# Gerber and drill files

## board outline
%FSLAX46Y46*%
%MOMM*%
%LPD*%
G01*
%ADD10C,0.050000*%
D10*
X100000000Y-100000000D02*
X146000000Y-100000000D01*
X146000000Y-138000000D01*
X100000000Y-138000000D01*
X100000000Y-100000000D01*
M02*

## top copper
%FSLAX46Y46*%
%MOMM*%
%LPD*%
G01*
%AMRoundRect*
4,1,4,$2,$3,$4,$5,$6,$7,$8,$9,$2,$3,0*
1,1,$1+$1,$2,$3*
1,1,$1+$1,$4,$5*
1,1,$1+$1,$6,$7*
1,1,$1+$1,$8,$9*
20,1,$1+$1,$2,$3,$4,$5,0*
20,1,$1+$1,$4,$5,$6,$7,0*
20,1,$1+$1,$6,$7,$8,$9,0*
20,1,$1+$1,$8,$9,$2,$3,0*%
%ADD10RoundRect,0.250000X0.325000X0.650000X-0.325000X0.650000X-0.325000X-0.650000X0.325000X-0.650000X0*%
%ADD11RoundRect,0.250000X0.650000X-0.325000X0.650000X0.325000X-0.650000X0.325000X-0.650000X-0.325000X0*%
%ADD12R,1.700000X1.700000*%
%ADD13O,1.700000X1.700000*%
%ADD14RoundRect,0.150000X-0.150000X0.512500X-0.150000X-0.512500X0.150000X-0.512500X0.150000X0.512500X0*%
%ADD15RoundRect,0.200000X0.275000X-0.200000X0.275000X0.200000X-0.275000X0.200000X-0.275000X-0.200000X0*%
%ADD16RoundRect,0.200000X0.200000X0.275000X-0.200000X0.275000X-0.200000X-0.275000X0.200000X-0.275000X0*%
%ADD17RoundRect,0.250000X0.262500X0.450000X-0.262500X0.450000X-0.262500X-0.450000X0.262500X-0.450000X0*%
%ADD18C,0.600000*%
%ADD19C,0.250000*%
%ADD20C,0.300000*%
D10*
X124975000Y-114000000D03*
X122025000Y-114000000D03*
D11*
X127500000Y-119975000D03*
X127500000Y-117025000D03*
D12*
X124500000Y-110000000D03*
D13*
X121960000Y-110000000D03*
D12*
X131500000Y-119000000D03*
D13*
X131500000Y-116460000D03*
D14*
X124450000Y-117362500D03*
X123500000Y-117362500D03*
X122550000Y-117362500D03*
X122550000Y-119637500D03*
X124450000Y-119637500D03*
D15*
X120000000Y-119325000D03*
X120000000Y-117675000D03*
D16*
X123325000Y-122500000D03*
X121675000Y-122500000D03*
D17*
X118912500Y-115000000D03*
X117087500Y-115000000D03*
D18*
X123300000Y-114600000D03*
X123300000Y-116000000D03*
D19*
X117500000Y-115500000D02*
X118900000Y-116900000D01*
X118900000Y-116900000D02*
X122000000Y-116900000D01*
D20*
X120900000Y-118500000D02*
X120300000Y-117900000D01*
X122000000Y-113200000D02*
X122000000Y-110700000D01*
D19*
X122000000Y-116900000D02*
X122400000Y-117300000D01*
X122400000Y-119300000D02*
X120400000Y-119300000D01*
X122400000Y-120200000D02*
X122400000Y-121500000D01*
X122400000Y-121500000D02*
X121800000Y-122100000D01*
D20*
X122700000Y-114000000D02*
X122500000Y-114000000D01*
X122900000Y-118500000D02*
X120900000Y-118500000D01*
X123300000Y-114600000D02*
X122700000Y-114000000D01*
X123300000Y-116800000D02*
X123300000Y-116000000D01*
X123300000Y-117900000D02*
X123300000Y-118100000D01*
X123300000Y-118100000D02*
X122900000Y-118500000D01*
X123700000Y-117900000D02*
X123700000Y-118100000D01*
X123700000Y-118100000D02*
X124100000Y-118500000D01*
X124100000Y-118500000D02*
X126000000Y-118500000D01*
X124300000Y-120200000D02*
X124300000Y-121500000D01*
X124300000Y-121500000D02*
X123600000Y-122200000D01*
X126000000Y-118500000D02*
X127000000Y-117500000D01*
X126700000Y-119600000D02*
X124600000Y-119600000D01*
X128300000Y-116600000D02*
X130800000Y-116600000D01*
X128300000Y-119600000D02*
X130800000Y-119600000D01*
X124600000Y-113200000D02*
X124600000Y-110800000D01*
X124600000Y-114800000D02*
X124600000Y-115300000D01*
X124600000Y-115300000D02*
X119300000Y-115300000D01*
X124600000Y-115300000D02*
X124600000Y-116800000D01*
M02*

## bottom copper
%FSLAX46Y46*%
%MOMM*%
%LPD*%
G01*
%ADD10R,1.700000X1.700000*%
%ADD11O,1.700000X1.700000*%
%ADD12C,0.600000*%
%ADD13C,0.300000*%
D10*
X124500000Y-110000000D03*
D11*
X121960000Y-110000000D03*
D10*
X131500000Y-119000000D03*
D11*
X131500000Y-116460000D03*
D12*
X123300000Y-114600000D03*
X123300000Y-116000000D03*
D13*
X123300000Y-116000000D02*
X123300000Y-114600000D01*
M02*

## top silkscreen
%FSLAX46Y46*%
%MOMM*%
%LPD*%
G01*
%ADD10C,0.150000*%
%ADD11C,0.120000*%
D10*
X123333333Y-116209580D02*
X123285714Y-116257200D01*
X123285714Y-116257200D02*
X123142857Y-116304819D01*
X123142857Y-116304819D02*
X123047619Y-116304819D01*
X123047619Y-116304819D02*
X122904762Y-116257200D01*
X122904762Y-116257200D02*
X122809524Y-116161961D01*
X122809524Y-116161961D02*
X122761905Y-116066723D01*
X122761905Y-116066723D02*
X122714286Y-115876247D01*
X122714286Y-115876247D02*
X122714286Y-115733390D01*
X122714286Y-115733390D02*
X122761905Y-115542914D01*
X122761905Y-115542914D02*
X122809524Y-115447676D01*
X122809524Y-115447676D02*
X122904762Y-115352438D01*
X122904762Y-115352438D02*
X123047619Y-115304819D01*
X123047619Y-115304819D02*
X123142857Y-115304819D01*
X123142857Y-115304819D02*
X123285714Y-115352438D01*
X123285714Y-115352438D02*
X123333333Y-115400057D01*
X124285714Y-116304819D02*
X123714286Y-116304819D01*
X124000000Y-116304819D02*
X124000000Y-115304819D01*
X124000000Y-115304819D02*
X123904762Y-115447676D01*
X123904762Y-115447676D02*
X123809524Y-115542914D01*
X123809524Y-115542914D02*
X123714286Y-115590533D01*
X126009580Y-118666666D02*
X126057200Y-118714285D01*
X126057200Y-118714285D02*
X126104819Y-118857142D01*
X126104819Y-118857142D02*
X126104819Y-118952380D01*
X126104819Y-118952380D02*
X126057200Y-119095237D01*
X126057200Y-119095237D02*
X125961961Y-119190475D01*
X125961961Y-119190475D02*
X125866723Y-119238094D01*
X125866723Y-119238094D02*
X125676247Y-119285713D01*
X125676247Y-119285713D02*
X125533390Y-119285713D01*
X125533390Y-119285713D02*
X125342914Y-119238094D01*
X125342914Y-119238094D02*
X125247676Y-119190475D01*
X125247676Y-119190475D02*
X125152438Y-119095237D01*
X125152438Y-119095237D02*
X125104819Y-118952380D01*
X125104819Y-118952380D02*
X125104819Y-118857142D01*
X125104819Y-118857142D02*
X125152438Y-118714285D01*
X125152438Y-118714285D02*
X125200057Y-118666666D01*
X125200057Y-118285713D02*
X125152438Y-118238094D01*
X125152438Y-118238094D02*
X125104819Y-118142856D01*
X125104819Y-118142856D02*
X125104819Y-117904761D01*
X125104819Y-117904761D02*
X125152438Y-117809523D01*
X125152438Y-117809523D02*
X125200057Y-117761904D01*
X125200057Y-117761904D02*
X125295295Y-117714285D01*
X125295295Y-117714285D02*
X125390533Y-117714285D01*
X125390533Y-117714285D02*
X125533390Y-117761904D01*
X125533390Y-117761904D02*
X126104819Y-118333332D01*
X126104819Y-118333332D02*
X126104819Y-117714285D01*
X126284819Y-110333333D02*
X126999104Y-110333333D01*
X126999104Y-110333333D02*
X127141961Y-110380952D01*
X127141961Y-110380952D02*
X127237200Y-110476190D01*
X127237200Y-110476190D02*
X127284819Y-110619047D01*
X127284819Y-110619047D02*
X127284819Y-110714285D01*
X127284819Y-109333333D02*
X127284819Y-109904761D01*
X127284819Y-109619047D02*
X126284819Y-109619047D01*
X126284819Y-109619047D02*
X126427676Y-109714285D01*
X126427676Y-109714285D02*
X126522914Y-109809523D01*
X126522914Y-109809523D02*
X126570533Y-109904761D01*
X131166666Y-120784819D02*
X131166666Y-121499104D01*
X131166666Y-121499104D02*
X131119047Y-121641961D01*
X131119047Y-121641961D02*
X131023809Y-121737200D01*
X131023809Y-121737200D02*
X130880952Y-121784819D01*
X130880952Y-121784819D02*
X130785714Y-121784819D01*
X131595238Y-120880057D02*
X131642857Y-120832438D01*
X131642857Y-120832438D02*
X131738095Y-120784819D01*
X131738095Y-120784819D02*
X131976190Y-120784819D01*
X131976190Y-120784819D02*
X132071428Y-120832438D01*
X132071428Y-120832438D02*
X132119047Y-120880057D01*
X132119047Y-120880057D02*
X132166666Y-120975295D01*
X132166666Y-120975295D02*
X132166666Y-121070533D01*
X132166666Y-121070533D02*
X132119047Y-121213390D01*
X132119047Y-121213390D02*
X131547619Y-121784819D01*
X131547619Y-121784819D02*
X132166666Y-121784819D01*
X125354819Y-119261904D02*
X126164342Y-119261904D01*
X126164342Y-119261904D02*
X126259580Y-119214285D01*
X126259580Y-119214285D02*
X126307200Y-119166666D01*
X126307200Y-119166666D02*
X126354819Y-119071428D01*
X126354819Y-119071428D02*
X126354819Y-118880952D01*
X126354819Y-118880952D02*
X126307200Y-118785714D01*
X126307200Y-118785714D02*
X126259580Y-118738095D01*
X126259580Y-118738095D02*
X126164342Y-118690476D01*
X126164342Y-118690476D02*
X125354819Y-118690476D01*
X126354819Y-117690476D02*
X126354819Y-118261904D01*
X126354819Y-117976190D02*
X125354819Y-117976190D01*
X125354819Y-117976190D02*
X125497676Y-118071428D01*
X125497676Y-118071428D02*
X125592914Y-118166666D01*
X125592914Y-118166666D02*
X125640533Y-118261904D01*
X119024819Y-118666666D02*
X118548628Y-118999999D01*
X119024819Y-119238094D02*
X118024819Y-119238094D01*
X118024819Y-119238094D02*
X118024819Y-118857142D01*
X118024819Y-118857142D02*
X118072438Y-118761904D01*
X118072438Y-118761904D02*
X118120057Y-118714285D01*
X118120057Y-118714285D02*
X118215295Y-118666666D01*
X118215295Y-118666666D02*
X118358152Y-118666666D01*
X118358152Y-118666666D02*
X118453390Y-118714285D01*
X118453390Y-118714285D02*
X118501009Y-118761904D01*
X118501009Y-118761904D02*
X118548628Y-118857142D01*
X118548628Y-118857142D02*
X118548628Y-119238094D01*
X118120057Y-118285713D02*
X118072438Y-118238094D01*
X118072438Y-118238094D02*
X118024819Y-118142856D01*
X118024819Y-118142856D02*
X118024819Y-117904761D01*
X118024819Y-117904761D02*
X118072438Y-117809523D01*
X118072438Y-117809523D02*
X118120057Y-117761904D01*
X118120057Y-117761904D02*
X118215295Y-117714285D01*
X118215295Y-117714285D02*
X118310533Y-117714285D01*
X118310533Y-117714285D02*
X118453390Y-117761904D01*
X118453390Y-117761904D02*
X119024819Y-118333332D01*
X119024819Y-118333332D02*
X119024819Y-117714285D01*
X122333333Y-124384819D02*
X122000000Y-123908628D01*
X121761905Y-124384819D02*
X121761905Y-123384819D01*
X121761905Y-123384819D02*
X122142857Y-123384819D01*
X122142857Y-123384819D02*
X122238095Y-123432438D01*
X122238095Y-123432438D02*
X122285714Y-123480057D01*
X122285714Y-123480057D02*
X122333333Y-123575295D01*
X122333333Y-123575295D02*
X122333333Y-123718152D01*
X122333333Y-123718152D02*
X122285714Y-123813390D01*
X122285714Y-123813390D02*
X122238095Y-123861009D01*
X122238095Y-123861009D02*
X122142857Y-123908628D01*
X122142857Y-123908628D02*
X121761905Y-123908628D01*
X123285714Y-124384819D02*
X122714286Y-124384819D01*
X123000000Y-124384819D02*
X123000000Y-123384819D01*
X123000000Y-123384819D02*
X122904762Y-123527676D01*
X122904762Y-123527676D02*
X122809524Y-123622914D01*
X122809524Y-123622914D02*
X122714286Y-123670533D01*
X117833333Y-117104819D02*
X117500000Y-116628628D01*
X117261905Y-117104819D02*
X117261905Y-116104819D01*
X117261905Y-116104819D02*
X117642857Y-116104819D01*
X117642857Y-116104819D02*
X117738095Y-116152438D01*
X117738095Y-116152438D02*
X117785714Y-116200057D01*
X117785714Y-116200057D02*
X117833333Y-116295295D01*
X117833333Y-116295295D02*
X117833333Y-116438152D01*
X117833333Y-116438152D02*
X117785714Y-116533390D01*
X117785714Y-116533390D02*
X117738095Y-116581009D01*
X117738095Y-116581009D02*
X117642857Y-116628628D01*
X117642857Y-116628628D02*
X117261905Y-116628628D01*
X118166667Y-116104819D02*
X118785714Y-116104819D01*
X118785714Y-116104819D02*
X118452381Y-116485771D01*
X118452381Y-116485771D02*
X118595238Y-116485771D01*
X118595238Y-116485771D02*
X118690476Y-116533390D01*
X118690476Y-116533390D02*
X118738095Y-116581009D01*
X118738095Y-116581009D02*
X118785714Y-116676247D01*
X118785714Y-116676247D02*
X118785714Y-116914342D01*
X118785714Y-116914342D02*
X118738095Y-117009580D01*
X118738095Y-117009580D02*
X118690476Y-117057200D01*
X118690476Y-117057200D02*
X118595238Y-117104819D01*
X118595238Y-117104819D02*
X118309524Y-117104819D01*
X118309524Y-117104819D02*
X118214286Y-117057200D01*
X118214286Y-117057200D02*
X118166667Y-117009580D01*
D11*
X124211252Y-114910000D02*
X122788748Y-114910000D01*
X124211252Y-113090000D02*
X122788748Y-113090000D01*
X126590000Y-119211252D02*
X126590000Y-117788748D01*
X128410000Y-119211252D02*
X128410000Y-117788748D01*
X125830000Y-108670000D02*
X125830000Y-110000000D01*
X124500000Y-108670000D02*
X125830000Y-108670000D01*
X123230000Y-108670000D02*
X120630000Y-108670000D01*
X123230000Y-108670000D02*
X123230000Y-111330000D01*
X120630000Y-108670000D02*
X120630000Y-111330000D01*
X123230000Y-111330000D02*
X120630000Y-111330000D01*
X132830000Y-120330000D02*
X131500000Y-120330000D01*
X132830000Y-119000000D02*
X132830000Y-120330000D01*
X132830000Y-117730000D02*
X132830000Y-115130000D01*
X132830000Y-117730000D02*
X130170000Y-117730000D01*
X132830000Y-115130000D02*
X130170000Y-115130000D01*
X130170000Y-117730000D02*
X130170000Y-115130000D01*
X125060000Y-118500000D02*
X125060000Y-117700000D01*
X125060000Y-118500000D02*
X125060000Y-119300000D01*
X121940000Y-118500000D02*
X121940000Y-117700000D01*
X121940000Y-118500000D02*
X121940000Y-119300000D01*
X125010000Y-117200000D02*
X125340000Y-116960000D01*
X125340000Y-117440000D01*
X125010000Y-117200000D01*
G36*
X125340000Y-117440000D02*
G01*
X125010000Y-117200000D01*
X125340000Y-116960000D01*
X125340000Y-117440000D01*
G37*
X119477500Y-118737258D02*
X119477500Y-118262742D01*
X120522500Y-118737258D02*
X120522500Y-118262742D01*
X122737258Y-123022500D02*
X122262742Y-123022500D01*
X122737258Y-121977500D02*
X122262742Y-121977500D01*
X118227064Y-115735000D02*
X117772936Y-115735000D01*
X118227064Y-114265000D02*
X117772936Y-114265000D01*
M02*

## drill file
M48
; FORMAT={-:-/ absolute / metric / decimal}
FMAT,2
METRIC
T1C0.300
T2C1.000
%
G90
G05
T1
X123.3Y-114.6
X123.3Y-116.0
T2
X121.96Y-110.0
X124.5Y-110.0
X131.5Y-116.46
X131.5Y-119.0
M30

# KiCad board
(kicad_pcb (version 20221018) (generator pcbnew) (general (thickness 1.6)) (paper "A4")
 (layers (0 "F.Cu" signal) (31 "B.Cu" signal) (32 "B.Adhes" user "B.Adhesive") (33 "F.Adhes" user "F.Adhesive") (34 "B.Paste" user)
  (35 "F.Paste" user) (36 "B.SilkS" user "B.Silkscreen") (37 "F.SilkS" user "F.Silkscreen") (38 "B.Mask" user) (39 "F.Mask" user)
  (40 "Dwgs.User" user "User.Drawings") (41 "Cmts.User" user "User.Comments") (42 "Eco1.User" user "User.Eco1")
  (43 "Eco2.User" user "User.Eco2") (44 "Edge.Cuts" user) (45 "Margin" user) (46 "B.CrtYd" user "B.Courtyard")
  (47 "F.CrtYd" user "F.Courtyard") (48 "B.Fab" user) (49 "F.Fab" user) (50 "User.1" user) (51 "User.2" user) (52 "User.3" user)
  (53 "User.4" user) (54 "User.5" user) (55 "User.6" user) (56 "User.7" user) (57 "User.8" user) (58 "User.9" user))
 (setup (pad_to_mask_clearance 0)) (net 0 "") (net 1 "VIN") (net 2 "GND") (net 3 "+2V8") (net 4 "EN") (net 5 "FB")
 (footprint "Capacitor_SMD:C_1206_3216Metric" (layer "F.Cu") (at 123.5 114 180)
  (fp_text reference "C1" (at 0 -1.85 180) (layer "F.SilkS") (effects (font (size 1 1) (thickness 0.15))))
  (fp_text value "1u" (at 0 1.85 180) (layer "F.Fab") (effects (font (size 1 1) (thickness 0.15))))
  (fp_line (start -0.711252 -0.91) (end 0.711252 -0.91) (stroke (width 0.12) (type solid)) (layer "F.SilkS"))
  (fp_line (start -0.711252 0.91) (end 0.711252 0.91) (stroke (width 0.12) (type solid)) (layer "F.SilkS"))
  (pad "1" smd roundrect (at -1.475 0 180) (size 1.15 1.8) (layers "F.Cu" "F.Paste" "F.Mask") (roundrect_rratio 0.217391) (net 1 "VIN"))
  (pad "2" smd roundrect (at 1.475 0 180) (size 1.15 1.8) (layers "F.Cu" "F.Paste" "F.Mask") (roundrect_rratio 0.217391) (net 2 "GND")))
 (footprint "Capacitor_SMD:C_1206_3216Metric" (layer "F.Cu") (at 127.5 118.5 90)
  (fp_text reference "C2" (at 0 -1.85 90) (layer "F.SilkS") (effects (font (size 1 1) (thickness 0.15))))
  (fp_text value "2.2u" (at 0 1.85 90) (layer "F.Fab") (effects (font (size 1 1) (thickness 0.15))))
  (fp_line (start -0.711252 -0.91) (end 0.711252 -0.91) (stroke (width 0.12) (type solid)) (layer "F.SilkS"))
  (fp_line (start -0.711252 0.91) (end 0.711252 0.91) (stroke (width 0.12) (type solid)) (layer "F.SilkS"))
  (pad "1" smd roundrect (at -1.475 0 90) (size 1.15 1.8) (layers "F.Cu" "F.Paste" "F.Mask") (roundrect_rratio 0.217391) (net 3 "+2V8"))
  (pad "2" smd roundrect (at 1.475 0 90) (size 1.15 1.8) (layers "F.Cu" "F.Paste" "F.Mask") (roundrect_rratio 0.217391) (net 2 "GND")))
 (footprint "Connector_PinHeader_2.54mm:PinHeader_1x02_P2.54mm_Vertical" (layer "F.Cu") (at 124.5 110 -90)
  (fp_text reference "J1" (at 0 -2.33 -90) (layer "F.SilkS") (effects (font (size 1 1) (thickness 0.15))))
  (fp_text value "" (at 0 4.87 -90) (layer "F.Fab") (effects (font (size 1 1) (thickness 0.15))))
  (fp_line (start -1.33 -1.33) (end 0 -1.33) (stroke (width 0.12) (type solid)) (layer "F.SilkS"))
  (fp_line (start -1.33 0) (end -1.33 -1.33) (stroke (width 0.12) (type solid)) (layer "F.SilkS"))
  (fp_line (start -1.33 1.27) (end -1.33 3.87) (stroke (width 0.12) (type solid)) (layer "F.SilkS"))
  (fp_line (start -1.33 1.27) (end 1.33 1.27) (stroke (width 0.12) (type solid)) (layer "F.SilkS"))
  (fp_line (start -1.33 3.87) (end 1.33 3.87) (stroke (width 0.12) (type solid)) (layer "F.SilkS"))
  (fp_line (start 1.33 1.27) (end 1.33 3.87) (stroke (width 0.12) (type solid)) (layer "F.SilkS"))
  (pad "1" thru_hole rect (at 0 0 270) (size 1.7 1.7) (drill 1) (layers "*.Cu" "*.Mask") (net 1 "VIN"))
  (pad "2" thru_hole oval (at 0 2.54 270) (size 1.7 1.7) (drill 1) (layers "*.Cu" "*.Mask") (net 2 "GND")))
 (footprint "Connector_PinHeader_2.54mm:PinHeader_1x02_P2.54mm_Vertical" (layer "F.Cu") (at 131.5 119 180)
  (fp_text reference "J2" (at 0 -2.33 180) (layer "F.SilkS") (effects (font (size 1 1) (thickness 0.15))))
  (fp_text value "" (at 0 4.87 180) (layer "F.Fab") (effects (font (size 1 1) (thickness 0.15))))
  (fp_line (start -1.33 -1.33) (end 0 -1.33) (stroke (width 0.12) (type solid)) (layer "F.SilkS"))
  (fp_line (start -1.33 0) (end -1.33 -1.33) (stroke (width 0.12) (type solid)) (layer "F.SilkS"))
  (fp_line (start -1.33 1.27) (end -1.33 3.87) (stroke (width 0.12) (type solid)) (layer "F.SilkS"))
  (fp_line (start -1.33 1.27) (end 1.33 1.27) (stroke (width 0.12) (type solid)) (layer "F.SilkS"))
  (fp_line (start -1.33 3.87) (end 1.33 3.87) (stroke (width 0.12) (type solid)) (layer "F.SilkS"))
  (fp_line (start 1.33 1.27) (end 1.33 3.87) (stroke (width 0.12) (type solid)) (layer "F.SilkS"))
  (pad "1" thru_hole rect (at 0 0 180) (size 1.7 1.7) (drill 1) (layers "*.Cu" "*.Mask") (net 3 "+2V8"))
  (pad "2" thru_hole oval (at 0 2.54 180) (size 1.7 1.7) (drill 1) (layers "*.Cu" "*.Mask") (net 2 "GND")))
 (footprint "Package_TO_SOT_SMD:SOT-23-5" (layer "F.Cu") (at 123.5 118.5 -90)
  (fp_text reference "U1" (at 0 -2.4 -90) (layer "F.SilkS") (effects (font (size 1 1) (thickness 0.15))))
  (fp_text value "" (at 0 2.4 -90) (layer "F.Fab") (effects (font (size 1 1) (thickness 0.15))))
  (fp_line (start 0 -1.56) (end -0.8 -1.56) (stroke (width 0.12) (type solid)) (layer "F.SilkS"))
  (fp_line (start 0 -1.56) (end 0.8 -1.56) (stroke (width 0.12) (type solid)) (layer "F.SilkS"))
  (fp_line (start 0 1.56) (end -0.8 1.56) (stroke (width 0.12) (type solid)) (layer "F.SilkS"))
  (fp_line (start 0 1.56) (end 0.8 1.56) (stroke (width 0.12) (type solid)) (layer "F.SilkS"))
  (fp_poly
   (pts (xy -1.3 -1.51) (xy -1.54 -1.84) (xy -1.06 -1.84) (xy -1.3 -1.51)) (stroke (width 0.12) (type solid)) (fill solid) (layer "F.SilkS"))
  (pad "1" smd roundrect (at -1.1375 -0.95 270) (size 1.325 0.6) (layers "F.Cu" "F.Paste" "F.Mask") (roundrect_rratio 0.25) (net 1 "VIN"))
  (pad "2" smd roundrect (at -1.1375 0 270) (size 1.325 0.6) (layers "F.Cu" "F.Paste" "F.Mask") (roundrect_rratio 0.25) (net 2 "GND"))
  (pad "3" smd roundrect (at -1.1375 0.95 270) (size 1.325 0.6) (layers "F.Cu" "F.Paste" "F.Mask") (roundrect_rratio 0.25) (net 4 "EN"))
  (pad "4" smd roundrect (at 1.1375 0.95 270) (size 1.325 0.6) (layers "F.Cu" "F.Paste" "F.Mask") (roundrect_rratio 0.25) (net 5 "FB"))
  (pad "5" smd roundrect (at 1.1375 -0.95 270) (size 1.325 0.6) (layers "F.Cu" "F.Paste" "F.Mask") (roundrect_rratio 0.25) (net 3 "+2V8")))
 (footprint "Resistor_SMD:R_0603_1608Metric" (layer "F.Cu") (at 120 118.5 90)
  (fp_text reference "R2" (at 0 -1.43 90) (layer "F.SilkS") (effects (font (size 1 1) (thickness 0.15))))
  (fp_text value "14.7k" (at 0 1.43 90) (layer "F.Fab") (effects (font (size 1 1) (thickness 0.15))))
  (fp_line (start -0.237258 -0.5225) (end 0.237258 -0.5225) (stroke (width 0.12) (type solid)) (layer "F.SilkS"))
  (fp_line (start -0.237258 0.5225) (end 0.237258 0.5225) (stroke (width 0.12) (type solid)) (layer "F.SilkS"))
  (pad "1" smd roundrect (at -0.825 0 90) (size 0.8 0.95) (layers "F.Cu" "F.Paste" "F.Mask") (roundrect_rratio 0.25) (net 5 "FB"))
  (pad "2" smd roundrect (at 0.825 0 90) (size 0.8 0.95) (layers "F.Cu" "F.Paste" "F.Mask") (roundrect_rratio 0.25) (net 2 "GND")))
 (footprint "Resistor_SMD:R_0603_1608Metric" (layer "F.Cu") (at 122.5 122.5 180)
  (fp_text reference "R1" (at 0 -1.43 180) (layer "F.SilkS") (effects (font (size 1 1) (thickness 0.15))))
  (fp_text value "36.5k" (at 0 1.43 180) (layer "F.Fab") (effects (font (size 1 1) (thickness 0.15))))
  (fp_line (start -0.237258 -0.5225) (end 0.237258 -0.5225) (stroke (width 0.12) (type solid)) (layer "F.SilkS"))
  (fp_line (start -0.237258 0.5225) (end 0.237258 0.5225) (stroke (width 0.12) (type solid)) (layer "F.SilkS"))
  (pad "1" smd roundrect (at -0.825 0 180) (size 0.8 0.95) (layers "F.Cu" "F.Paste" "F.Mask") (roundrect_rratio 0.25) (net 3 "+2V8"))
  (pad "2" smd roundrect (at 0.825 0 180) (size 0.8 0.95) (layers "F.Cu" "F.Paste" "F.Mask") (roundrect_rratio 0.25) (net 5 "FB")))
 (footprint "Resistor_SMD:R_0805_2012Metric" (layer "F.Cu") (at 118 115 180)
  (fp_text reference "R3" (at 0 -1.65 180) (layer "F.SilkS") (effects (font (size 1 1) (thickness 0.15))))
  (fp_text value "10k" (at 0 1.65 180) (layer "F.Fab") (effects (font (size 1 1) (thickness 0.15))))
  (fp_line (start -0.227064 -0.735) (end 0.227064 -0.735) (stroke (width 0.12) (type solid)) (layer "F.SilkS"))
  (fp_line (start -0.227064 0.735) (end 0.227064 0.735) (stroke (width 0.12) (type solid)) (layer "F.SilkS"))
  (pad "1" smd roundrect (at -0.9125 0 180) (size 1.025 1.4) (layers "F.Cu" "F.Paste" "F.Mask") (roundrect_rratio 0.243902) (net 1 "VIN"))
  (pad "2" smd roundrect (at 0.9125 0 180) (size 1.025 1.4) (layers "F.Cu" "F.Paste" "F.Mask") (roundrect_rratio 0.243902) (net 4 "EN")))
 (gr_rect (start 100 100) (end 146 138) (stroke (width 0.05) (type default)) (fill none) (layer "Edge.Cuts"))
 (segment (start 117.5 115.5) (end 118.9 116.9) (width 0.25) (layer "F.Cu") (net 4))
 (segment (start 118.9 116.9) (end 122 116.9) (width 0.25) (layer "F.Cu") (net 4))
 (segment (start 120.9 118.5) (end 120.3 117.9) (width 0.3) (layer "F.Cu") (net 2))
 (segment (start 122 113.2) (end 122 110.7) (width 0.3) (layer "F.Cu") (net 2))
 (segment (start 122 116.9) (end 122.4 117.3) (width 0.25) (layer "F.Cu") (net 4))
 (segment (start 122.4 119.3) (end 120.4 119.3) (width 0.25) (layer "F.Cu") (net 5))
 (segment (start 122.4 120.2) (end 122.4 121.5) (width 0.25) (layer "F.Cu") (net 5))
 (segment (start 122.4 121.5) (end 121.8 122.1) (width 0.25) (layer "F.Cu") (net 5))
 (segment (start 122.7 114) (end 122.5 114) (width 0.3) (layer "F.Cu") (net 2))
 (segment (start 122.9 118.5) (end 120.9 118.5) (width 0.3) (layer "F.Cu") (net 2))
 (segment (start 123.3 114.6) (end 122.7 114) (width 0.3) (layer "F.Cu") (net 2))
 (segment (start 123.3 116.8) (end 123.3 116) (width 0.3) (layer "F.Cu") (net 2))
 (segment (start 123.3 117.9) (end 123.3 118.1) (width 0.3) (layer "F.Cu") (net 2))
 (segment (start 123.3 118.1) (end 122.9 118.5) (width 0.3) (layer "F.Cu") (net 2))
 (segment (start 123.7 117.9) (end 123.7 118.1) (width 0.3) (layer "F.Cu") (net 2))
 (segment (start 123.7 118.1) (end 124.1 118.5) (width 0.3) (layer "F.Cu") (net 2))
 (segment (start 124.1 118.5) (end 126 118.5) (width 0.3) (layer "F.Cu") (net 2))
 (segment (start 124.3 120.2) (end 124.3 121.5) (width 0.3) (layer "F.Cu") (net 3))
 (segment (start 124.3 121.5) (end 123.6 122.2) (width 0.3) (layer "F.Cu") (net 3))
 (segment (start 126 118.5) (end 127 117.5) (width 0.3) (layer "F.Cu") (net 2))
 (segment (start 126.7 119.6) (end 124.6 119.6) (width 0.3) (layer "F.Cu") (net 3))
 (segment (start 128.3 116.6) (end 130.8 116.6) (width 0.3) (layer "F.Cu") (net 2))
 (segment (start 128.3 119.6) (end 130.8 119.6) (width 0.3) (layer "F.Cu") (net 3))
 (via (at 123.3 114.6) (size 0.6) (drill 0.3) (layers "F.Cu" "B.Cu") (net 2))
 (via (at 123.3 116) (size 0.6) (drill 0.3) (layers "F.Cu" "B.Cu") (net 2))
 (segment (start 123.3 116) (end 123.3 114.6) (width 0.3) (layer "B.Cu") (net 2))
 (segment (start 124.6 113.2) (end 124.6 110.8) (width 0.3) (layer "F.Cu") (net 1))
 (segment (start 124.6 114.8) (end 124.6 115.3) (width 0.3) (layer "F.Cu") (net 1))
 (segment (start 124.6 115.3) (end 119.3 115.3) (width 0.3) (layer "F.Cu") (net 1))
 (segment (start 124.6 115.3) (end 124.6 116.8) (width 0.3) (layer "F.Cu") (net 1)))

